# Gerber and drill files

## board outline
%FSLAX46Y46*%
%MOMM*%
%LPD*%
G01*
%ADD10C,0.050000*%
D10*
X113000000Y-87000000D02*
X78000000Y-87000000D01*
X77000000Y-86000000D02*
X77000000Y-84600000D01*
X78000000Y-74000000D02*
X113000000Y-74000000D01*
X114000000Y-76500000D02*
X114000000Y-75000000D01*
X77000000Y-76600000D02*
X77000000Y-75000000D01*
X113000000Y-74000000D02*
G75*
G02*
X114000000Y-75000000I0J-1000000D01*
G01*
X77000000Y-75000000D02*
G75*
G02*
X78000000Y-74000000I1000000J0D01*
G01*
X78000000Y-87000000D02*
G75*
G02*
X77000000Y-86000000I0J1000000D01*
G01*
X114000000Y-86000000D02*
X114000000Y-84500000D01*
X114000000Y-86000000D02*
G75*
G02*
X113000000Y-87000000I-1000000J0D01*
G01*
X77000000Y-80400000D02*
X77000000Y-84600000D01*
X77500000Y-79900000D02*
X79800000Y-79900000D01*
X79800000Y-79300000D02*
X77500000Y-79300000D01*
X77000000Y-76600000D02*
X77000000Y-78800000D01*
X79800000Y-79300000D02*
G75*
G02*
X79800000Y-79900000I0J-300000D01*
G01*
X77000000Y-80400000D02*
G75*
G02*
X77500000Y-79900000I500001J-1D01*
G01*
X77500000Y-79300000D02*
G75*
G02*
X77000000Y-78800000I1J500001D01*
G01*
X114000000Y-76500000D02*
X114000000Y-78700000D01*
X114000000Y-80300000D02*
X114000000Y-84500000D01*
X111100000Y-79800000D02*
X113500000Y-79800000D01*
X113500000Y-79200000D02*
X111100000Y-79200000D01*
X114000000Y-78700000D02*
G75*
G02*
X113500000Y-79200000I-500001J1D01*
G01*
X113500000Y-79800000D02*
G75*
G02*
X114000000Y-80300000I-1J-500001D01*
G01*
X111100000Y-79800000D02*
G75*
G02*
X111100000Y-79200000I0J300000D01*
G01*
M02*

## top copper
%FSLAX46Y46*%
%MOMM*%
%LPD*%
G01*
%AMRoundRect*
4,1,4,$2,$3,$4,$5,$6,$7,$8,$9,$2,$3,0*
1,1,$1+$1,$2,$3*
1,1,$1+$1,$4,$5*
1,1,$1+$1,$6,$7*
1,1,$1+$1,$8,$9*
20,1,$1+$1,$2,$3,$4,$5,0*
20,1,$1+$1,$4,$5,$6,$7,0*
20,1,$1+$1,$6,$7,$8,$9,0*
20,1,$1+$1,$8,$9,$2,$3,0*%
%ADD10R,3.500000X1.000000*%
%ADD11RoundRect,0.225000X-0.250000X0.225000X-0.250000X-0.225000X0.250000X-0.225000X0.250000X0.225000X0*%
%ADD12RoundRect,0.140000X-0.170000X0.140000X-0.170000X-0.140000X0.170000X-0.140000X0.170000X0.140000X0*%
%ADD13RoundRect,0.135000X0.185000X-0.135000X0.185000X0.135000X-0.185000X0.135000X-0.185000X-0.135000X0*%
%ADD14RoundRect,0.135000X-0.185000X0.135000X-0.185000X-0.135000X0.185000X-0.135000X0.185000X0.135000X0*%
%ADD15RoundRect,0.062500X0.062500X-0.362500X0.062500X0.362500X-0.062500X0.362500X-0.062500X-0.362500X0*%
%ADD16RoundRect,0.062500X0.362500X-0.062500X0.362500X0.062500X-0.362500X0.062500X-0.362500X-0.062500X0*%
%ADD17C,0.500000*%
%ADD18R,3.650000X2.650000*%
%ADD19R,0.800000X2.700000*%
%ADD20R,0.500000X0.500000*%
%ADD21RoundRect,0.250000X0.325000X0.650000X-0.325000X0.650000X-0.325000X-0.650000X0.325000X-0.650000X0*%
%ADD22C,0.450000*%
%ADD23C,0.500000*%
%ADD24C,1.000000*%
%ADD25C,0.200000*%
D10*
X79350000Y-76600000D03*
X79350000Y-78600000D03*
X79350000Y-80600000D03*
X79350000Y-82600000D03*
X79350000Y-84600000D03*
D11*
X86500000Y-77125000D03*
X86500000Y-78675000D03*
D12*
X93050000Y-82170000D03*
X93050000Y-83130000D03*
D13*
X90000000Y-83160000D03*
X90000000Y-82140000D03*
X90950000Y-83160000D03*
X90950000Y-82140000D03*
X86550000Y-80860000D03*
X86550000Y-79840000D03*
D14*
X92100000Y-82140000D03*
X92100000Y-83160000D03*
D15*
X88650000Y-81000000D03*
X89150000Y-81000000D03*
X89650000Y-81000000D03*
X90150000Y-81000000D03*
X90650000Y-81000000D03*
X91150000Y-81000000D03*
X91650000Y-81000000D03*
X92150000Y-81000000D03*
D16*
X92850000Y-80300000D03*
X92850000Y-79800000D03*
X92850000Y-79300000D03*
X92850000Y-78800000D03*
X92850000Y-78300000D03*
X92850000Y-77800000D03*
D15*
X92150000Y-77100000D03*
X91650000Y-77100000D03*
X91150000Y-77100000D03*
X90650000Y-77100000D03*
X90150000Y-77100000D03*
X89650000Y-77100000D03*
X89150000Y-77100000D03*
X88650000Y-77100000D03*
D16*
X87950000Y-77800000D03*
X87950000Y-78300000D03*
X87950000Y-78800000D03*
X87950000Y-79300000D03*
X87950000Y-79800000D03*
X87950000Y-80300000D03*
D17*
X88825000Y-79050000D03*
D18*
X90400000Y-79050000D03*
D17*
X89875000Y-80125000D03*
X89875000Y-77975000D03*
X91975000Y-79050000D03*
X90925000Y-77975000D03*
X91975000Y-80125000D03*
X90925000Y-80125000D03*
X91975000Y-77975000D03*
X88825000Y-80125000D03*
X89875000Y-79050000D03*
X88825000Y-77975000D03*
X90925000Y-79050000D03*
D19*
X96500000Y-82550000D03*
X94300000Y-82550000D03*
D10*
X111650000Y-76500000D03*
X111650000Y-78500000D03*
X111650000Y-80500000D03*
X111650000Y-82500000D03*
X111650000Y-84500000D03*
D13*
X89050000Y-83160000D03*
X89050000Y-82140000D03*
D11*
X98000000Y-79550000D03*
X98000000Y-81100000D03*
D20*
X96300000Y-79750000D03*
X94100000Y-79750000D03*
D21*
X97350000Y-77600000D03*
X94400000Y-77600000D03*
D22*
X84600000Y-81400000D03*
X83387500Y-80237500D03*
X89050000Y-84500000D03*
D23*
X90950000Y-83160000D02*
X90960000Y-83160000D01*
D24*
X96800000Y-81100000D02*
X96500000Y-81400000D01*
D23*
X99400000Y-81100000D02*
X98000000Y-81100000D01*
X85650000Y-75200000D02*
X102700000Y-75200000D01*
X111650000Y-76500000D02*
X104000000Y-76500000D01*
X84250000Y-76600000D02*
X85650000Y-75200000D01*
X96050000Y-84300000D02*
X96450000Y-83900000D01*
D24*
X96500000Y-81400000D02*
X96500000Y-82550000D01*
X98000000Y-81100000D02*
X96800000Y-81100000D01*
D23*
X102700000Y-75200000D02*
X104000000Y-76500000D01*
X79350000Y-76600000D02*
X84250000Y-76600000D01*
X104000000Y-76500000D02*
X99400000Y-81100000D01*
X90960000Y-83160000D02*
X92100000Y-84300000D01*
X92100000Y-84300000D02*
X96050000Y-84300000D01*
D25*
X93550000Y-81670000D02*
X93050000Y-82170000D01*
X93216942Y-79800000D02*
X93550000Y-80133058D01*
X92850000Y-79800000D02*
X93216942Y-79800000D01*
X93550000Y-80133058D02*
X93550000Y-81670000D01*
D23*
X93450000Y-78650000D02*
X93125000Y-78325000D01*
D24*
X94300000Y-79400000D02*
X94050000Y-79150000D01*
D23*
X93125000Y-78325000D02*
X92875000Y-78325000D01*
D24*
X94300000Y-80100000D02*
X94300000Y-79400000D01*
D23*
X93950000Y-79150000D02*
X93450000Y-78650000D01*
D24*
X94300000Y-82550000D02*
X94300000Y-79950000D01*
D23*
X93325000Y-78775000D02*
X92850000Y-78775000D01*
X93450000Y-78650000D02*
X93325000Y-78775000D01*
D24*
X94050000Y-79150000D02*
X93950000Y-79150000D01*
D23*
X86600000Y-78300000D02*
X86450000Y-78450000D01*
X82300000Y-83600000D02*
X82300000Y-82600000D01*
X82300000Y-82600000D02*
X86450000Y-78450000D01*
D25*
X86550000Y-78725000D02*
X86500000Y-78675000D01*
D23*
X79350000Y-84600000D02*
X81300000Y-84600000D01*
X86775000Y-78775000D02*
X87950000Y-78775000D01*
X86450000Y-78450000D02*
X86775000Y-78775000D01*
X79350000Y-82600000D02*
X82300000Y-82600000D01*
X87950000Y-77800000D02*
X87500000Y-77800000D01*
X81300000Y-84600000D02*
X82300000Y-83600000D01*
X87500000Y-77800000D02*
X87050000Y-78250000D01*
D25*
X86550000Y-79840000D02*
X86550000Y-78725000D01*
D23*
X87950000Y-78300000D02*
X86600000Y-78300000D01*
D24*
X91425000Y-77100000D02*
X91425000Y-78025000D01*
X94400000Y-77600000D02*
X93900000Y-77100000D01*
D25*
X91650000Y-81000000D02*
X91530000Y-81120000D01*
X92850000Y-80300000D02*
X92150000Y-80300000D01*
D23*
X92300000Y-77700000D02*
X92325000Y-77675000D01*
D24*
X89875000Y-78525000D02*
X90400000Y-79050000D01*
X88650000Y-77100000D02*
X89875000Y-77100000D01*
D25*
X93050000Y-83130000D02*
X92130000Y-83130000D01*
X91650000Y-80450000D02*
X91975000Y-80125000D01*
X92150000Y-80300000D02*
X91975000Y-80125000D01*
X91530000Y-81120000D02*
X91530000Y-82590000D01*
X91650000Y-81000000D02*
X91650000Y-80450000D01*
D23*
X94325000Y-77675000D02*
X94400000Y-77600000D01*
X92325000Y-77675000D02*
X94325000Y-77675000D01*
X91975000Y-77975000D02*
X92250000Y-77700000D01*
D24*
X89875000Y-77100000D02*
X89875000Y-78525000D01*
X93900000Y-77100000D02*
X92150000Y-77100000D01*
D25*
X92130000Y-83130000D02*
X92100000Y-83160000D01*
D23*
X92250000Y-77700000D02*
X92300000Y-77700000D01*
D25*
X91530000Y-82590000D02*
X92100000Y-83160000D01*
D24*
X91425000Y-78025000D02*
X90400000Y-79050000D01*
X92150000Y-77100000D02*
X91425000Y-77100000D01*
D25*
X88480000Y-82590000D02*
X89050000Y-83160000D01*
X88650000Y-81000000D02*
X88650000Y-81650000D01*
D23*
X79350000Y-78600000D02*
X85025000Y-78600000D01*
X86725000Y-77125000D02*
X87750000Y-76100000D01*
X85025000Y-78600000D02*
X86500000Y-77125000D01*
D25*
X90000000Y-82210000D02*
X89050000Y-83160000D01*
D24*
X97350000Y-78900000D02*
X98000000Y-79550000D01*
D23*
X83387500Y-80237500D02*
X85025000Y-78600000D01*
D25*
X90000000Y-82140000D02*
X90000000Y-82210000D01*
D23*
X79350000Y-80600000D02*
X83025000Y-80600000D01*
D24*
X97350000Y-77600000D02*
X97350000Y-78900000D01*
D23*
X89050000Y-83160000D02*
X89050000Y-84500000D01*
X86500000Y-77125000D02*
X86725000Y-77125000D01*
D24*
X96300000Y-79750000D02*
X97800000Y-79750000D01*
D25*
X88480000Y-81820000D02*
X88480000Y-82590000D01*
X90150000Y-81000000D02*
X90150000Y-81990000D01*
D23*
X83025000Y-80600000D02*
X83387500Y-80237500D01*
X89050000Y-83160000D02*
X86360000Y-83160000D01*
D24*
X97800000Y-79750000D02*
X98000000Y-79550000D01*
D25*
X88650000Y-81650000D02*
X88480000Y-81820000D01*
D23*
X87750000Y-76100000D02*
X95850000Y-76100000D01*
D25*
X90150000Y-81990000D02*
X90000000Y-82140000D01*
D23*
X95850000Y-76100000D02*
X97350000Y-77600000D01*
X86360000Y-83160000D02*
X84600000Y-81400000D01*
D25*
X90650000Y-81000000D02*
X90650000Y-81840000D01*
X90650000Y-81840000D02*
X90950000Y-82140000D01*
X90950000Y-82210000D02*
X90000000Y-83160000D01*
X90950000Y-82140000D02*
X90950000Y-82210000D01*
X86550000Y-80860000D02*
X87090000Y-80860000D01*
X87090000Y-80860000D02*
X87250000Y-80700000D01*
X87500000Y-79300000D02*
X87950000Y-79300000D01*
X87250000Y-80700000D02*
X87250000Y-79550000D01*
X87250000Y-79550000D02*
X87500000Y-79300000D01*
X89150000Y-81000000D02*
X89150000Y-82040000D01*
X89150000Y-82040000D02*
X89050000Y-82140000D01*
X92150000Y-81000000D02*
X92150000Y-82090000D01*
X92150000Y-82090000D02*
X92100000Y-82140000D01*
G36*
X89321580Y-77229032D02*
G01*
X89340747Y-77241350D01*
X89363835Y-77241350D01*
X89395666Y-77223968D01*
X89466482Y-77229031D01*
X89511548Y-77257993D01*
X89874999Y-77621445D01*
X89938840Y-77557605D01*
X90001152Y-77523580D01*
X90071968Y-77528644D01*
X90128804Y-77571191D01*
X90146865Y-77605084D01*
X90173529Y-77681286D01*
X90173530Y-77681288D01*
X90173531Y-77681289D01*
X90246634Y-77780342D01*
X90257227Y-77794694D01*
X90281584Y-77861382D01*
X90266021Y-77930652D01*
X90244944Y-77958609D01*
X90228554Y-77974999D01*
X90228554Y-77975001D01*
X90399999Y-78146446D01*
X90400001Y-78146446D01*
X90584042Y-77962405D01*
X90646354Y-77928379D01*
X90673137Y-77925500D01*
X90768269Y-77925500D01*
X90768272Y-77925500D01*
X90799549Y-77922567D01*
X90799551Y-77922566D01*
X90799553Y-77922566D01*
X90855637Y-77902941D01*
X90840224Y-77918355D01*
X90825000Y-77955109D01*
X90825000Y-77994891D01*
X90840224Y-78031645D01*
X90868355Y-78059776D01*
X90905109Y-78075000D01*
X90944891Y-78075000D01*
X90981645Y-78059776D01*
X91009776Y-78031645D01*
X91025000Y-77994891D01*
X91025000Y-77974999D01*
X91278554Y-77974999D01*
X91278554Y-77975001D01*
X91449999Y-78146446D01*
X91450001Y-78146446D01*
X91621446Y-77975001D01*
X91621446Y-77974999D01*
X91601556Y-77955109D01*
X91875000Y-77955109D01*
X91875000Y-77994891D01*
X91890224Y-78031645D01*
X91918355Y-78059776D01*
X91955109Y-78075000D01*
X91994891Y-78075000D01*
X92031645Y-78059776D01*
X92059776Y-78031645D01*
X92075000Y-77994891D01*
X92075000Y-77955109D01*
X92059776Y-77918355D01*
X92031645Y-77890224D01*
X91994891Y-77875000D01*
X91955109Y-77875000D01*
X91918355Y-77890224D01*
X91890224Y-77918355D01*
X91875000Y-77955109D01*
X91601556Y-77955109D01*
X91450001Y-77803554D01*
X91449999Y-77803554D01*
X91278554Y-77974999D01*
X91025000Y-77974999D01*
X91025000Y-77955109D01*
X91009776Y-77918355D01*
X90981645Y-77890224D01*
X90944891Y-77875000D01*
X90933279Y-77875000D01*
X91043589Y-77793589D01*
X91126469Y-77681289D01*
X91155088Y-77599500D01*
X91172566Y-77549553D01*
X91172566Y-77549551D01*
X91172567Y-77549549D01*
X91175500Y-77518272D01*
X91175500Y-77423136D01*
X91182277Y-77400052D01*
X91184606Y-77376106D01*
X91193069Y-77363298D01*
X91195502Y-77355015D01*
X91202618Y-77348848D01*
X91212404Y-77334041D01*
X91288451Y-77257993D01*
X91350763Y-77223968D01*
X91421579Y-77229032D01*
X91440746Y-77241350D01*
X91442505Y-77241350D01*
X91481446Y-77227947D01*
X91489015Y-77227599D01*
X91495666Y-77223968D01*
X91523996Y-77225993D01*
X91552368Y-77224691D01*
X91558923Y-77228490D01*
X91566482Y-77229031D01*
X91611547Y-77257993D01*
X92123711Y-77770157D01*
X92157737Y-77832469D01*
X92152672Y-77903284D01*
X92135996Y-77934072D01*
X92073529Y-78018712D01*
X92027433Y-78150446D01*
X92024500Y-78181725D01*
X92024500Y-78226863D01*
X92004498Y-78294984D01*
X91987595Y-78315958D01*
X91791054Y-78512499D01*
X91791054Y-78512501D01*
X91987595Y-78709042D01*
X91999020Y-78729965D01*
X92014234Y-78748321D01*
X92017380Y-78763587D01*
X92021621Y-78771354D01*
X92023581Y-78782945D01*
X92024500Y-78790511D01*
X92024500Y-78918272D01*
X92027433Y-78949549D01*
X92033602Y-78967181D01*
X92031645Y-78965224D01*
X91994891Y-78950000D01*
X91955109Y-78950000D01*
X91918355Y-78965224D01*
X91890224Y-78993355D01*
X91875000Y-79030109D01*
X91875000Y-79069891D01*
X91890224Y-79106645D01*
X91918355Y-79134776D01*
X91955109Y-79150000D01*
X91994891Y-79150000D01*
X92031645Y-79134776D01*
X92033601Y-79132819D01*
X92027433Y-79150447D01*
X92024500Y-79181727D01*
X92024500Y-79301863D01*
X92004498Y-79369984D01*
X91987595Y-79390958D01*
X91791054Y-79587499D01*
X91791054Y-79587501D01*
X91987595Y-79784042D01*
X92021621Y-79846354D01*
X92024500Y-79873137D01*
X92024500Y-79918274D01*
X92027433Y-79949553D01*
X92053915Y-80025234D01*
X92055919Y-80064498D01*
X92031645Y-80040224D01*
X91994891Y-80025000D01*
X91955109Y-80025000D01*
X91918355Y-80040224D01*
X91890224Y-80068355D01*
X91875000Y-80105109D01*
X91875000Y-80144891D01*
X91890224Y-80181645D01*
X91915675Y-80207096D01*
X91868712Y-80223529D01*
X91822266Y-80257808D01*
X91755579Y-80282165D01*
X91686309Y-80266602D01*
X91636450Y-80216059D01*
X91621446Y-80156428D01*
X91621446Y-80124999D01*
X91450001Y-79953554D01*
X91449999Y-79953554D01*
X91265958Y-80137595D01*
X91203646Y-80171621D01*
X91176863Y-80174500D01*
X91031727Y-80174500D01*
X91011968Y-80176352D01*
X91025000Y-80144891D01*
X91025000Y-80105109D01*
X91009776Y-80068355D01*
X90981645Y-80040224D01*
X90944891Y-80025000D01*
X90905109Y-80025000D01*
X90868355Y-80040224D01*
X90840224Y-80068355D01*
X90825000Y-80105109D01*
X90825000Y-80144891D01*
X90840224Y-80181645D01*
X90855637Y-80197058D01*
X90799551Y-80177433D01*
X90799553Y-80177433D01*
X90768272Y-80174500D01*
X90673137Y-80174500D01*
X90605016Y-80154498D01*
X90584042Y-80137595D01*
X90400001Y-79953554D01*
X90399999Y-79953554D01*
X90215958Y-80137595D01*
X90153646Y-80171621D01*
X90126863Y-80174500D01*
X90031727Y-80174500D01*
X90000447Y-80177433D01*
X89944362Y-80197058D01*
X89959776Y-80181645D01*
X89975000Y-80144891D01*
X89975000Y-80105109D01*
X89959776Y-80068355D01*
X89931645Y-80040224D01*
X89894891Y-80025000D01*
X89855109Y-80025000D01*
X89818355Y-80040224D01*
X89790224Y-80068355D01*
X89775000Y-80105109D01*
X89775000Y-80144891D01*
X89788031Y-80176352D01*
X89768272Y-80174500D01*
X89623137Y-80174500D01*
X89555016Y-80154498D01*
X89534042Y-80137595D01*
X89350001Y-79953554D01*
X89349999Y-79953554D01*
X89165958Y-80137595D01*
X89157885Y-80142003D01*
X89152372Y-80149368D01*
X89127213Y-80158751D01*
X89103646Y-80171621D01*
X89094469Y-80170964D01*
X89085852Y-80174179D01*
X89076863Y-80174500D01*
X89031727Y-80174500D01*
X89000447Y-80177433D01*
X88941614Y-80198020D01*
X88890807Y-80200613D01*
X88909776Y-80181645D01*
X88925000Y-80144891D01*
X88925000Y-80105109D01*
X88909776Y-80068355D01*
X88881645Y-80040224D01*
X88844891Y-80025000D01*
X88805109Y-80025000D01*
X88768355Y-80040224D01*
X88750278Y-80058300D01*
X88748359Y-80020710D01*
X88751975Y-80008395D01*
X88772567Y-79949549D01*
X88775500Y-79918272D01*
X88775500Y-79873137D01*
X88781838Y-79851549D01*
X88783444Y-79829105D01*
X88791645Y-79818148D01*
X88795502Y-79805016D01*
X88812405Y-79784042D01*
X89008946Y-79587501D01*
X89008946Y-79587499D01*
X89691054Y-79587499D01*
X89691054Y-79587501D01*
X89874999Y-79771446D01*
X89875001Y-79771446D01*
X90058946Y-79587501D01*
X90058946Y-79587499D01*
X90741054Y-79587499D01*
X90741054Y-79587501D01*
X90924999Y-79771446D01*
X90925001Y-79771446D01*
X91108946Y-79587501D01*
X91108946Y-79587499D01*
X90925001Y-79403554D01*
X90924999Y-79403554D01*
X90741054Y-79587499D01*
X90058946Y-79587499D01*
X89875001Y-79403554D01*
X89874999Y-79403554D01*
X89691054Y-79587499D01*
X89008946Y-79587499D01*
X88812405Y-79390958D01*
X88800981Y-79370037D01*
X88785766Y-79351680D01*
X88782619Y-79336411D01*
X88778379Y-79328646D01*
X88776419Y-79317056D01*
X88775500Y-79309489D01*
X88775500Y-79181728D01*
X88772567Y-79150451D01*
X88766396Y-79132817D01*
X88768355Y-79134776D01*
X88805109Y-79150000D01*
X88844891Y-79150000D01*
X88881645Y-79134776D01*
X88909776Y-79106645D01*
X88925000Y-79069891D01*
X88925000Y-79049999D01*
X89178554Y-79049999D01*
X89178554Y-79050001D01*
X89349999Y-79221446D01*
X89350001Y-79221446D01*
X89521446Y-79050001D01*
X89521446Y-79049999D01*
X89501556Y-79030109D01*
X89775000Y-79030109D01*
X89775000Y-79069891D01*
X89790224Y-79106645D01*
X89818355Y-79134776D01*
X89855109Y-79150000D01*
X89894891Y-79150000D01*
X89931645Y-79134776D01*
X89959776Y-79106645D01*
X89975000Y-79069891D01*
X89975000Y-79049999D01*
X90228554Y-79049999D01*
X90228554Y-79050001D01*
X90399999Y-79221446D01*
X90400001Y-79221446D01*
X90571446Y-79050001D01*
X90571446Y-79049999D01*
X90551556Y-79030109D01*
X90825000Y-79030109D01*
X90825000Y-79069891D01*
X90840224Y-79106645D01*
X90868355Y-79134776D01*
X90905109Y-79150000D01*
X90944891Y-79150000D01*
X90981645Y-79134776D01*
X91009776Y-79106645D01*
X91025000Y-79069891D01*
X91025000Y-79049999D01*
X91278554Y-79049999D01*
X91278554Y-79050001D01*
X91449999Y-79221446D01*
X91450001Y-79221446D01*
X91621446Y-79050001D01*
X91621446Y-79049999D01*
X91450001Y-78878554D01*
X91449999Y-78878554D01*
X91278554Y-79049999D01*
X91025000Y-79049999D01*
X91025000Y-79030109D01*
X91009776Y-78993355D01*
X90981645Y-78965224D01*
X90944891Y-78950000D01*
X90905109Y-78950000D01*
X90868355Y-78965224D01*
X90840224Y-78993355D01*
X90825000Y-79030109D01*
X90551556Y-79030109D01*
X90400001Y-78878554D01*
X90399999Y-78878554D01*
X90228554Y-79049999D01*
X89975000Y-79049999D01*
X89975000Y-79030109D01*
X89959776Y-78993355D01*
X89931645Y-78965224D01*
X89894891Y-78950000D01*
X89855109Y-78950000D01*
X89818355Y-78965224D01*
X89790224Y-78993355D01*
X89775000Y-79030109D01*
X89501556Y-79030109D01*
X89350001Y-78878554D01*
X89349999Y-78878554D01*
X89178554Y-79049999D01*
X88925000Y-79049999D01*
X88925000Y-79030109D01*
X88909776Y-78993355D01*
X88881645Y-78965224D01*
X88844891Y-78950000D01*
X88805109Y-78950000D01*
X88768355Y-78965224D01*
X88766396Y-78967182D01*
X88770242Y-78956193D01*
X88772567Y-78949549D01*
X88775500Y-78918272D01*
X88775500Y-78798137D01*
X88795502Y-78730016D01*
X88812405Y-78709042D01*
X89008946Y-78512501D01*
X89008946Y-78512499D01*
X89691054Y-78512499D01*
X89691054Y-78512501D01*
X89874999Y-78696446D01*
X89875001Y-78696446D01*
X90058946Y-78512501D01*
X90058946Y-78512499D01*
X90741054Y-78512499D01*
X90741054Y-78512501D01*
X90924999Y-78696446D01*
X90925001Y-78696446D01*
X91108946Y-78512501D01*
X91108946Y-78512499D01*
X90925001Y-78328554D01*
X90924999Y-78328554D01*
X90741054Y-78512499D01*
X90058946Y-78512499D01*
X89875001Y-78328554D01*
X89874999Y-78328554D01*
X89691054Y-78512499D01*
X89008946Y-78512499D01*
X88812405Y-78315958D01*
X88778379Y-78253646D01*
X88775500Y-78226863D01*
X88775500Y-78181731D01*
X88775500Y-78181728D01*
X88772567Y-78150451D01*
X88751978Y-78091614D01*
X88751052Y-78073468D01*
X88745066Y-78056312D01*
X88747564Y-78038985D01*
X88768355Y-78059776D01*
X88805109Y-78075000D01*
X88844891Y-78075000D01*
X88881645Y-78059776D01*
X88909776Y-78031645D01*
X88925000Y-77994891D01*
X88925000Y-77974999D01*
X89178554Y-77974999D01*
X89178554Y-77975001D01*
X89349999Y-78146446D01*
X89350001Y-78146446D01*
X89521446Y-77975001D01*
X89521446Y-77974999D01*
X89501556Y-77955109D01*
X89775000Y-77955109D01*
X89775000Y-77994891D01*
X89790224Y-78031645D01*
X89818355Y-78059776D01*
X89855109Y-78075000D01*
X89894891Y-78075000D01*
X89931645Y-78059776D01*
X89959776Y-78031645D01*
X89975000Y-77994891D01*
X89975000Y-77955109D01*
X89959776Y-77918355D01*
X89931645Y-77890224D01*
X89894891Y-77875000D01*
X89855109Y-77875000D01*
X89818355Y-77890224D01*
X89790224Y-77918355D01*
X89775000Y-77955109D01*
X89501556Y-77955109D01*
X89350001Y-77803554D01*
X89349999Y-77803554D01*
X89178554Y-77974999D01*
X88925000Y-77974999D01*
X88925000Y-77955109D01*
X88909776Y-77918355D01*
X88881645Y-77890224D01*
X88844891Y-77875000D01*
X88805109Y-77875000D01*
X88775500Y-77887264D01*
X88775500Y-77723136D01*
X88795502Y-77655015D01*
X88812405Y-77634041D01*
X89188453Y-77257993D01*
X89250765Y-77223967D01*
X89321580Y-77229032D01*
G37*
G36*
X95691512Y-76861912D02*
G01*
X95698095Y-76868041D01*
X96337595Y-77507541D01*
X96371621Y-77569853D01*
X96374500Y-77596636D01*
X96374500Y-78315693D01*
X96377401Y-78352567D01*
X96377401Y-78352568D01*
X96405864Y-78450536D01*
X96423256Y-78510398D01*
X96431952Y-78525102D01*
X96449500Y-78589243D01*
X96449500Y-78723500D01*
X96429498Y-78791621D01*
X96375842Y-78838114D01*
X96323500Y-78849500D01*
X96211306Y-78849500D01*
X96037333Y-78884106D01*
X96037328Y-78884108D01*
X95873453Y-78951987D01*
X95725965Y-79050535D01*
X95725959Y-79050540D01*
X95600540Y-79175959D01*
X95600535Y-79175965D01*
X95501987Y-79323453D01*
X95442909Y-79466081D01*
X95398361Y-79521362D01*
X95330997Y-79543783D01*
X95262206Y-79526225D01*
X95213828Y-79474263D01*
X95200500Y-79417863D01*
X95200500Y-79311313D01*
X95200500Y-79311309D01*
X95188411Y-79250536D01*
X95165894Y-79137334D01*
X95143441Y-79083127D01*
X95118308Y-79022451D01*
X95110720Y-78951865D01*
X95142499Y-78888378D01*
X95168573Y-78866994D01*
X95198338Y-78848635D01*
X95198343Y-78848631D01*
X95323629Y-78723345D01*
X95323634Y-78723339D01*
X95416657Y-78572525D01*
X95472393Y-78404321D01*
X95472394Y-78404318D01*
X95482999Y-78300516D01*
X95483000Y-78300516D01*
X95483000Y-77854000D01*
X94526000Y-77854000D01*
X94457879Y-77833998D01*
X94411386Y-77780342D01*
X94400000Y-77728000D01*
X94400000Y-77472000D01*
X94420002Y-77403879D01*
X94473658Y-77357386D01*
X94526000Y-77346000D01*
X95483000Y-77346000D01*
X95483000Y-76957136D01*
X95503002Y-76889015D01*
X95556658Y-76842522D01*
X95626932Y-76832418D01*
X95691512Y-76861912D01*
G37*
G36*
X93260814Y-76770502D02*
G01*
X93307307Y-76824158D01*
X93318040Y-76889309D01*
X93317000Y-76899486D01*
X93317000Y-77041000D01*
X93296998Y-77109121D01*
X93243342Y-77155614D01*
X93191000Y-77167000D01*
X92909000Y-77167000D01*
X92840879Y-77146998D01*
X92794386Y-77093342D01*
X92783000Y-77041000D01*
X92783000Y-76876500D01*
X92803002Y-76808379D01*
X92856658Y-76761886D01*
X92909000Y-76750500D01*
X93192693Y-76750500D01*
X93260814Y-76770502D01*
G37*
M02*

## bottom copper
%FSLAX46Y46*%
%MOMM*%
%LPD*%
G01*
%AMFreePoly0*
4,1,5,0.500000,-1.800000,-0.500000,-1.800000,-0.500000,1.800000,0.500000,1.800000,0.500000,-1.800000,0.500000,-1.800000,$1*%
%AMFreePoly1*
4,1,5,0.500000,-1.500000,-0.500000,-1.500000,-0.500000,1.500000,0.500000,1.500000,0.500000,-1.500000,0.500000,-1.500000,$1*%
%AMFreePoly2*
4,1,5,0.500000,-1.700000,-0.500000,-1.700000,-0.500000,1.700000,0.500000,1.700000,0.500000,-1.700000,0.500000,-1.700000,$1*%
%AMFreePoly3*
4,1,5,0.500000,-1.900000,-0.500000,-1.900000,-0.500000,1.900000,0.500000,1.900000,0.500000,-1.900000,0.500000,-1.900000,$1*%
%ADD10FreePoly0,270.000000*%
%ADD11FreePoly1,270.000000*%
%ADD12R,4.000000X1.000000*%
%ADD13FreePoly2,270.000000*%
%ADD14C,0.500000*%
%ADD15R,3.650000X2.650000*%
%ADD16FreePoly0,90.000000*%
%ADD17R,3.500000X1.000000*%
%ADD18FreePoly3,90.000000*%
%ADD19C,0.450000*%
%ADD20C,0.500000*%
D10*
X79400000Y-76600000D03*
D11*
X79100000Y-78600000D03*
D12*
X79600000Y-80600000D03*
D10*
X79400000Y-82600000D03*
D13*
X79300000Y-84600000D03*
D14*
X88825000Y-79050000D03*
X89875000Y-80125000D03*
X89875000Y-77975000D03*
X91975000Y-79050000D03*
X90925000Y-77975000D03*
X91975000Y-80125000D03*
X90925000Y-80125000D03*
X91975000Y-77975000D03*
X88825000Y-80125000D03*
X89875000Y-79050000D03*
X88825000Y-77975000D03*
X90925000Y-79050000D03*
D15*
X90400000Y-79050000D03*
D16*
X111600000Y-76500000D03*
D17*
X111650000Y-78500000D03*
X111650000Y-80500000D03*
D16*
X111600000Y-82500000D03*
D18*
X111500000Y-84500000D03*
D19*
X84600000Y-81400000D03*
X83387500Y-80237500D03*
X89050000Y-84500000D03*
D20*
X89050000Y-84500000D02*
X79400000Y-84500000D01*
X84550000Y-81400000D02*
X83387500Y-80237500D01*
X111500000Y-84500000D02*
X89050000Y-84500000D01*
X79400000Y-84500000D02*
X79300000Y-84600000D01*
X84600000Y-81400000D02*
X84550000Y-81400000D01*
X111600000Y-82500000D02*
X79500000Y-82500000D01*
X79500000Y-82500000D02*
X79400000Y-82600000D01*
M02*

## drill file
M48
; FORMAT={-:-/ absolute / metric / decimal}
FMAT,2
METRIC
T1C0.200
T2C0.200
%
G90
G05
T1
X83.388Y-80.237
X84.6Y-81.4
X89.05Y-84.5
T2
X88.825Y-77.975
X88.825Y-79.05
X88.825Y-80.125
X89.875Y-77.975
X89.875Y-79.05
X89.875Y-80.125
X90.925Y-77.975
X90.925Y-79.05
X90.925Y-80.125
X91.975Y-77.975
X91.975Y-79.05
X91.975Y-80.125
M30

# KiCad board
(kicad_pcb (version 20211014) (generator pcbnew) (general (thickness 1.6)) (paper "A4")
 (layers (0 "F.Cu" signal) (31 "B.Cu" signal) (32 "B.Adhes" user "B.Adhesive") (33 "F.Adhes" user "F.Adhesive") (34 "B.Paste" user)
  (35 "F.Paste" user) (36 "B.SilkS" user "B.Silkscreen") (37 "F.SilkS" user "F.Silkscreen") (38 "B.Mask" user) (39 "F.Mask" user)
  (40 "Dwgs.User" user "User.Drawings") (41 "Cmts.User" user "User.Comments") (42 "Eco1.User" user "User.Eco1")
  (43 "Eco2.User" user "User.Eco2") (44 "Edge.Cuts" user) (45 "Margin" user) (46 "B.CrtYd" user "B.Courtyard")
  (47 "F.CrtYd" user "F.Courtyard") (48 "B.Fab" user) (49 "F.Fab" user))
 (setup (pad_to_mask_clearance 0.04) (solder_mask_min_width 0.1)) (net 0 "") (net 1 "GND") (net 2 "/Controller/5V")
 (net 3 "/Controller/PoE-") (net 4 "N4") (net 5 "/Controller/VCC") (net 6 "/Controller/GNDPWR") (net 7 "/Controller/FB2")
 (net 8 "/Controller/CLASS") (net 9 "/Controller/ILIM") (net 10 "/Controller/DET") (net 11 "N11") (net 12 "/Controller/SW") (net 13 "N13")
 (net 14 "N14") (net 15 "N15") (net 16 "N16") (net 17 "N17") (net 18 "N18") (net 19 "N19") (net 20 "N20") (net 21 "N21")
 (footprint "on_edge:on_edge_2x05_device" (layer "F.Cu") (at 77 80.6 -90)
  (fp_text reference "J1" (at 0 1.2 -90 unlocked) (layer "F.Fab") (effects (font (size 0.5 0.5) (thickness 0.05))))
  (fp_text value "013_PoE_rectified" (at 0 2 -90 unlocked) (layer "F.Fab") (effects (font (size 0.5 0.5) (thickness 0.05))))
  (fp_line (start -0.2 0) (end 4 0) (layer "Edge.Cuts") (width 0.05))
  (fp_line (start -0.7 -0.5) (end -0.7 -2.8) (layer "Edge.Cuts") (width 0.05))
  (fp_line (start -1.3 -2.8) (end -1.3 -0.5) (layer "Edge.Cuts") (width 0.05))
  (fp_line (start -4 0) (end -1.8 0) (layer "Edge.Cuts") (width 0.05))
  (fp_arc (start -1.3 -2.8) (mid -1 -3.1) (end -0.7 -2.8) (layer "Edge.Cuts") (width 0.05))
  (fp_arc (start -0.2 0) (mid -0.553553 -0.146447) (end -0.7 -0.5) (layer "Edge.Cuts") (width 0.05))
  (fp_arc (start -1.3 -0.5) (mid -1.446447 -0.146447) (end -1.8 0) (layer "Edge.Cuts") (width 0.05))
  (pad "1" smd rect (at -4 -2.35 90) (size 1 3.5) (layers "F.Cu" "F.Mask") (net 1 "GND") (zone_connect 0))
  (pad "2" smd rect (at -2 -2.35 270) (size 1 3.5) (layers "F.Cu" "F.Mask") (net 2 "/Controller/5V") (zone_connect 0))
  (pad "3" smd rect (at 0 -2.35 270) (size 1 3.5) (layers "F.Cu" "F.Mask") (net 2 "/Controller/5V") (zone_connect 0))
  (pad "4" smd rect (at 2 -2.35 90) (size 1 3.5) (layers "F.Cu" "F.Mask") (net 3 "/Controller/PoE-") (zone_connect 0))
  (pad "5" smd rect (at 4 -2.35 90) (size 1 3.5) (layers "F.Cu" "F.Mask") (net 3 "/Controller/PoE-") (zone_connect 0))
  (pad "6" smd custom (at -4 -2.4 270) (size 1 3.6) (layers "B.Cu" "B.Mask") (zone_connect 0) (options (clearance outline) (anchor rect))
   (primitives))
  (pad "7" smd custom (at -2 -2.1 270) (size 1 3) (layers "B.Cu" "B.Mask") (zone_connect 0) (options (clearance outline) (anchor rect))
   (primitives))
  (pad "8" smd rect (at 0 -2.6 270) (size 1 4) (layers "B.Cu" "B.Mask") (zone_connect 0))
  (pad "9" smd custom (at 2 -2.4 270) (size 1 3.6) (layers "B.Cu" "B.Mask") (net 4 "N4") (zone_connect 0)
   (options (clearance outline) (anchor rect)) (primitives))
  (pad "10" smd custom (at 4 -2.3 270) (size 1 3.4) (layers "B.Cu" "B.Mask") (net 2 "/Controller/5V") (zone_connect 0)
   (options (clearance outline) (anchor rect)) (primitives))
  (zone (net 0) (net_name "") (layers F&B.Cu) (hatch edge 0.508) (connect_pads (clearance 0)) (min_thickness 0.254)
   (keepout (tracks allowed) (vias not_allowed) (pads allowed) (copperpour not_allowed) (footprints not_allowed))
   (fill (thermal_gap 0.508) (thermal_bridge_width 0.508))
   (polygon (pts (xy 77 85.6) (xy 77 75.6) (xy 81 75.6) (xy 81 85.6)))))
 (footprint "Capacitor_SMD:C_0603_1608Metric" (layer "F.Cu") (at 86.5 77.9 -90)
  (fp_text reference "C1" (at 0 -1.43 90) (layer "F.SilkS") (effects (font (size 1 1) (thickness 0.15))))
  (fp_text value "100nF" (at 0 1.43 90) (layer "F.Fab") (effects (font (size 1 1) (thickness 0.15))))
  (pad "1" smd roundrect (at -0.775 0 270) (size 0.9 0.95) (layers "F.Cu" "F.Paste" "F.Mask") (roundrect_rratio 0.25)
   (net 2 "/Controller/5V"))
  (pad "2" smd roundrect (at 0.775 0 270) (size 0.9 0.95) (layers "F.Cu" "F.Paste" "F.Mask") (roundrect_rratio 0.25)
   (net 3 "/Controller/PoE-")))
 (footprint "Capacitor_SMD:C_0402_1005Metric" (layer "F.Cu") (at 93.05 82.65 -90)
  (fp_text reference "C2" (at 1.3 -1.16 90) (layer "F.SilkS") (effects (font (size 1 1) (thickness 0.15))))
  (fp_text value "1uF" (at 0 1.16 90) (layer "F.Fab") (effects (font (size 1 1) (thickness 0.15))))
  (pad "1" smd roundrect (at -0.48 0 270) (size 0.56 0.62) (layers "F.Cu" "F.Paste" "F.Mask") (roundrect_rratio 0.25)
   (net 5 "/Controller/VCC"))
  (pad "2" smd roundrect (at 0.48 0 270) (size 0.56 0.62) (layers "F.Cu" "F.Paste" "F.Mask") (roundrect_rratio 0.25)
   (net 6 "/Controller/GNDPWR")))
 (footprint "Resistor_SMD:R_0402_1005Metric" (layer "F.Cu") (at 90 82.65 90)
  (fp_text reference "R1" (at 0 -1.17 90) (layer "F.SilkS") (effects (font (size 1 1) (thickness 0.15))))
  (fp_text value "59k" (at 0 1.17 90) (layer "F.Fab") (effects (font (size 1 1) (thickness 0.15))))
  (pad "1" smd roundrect (at -0.51 0 90) (size 0.54 0.64) (layers "F.Cu" "F.Paste" "F.Mask") (roundrect_rratio 0.25)
   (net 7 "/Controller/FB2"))
  (pad "2" smd roundrect (at 0.51 0 90) (size 0.54 0.64) (layers "F.Cu" "F.Paste" "F.Mask") (roundrect_rratio 0.25) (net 2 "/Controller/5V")))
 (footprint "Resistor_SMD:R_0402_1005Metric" (layer "F.Cu") (at 90.95 82.65 90)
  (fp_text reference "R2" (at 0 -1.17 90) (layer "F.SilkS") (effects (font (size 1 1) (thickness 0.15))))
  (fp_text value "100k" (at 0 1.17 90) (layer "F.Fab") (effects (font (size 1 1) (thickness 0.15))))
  (pad "1" smd roundrect (at -0.51 0 90) (size 0.54 0.64) (layers "F.Cu" "F.Paste" "F.Mask") (roundrect_rratio 0.25) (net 1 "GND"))
  (pad "2" smd roundrect (at 0.51 0 90) (size 0.54 0.64) (layers "F.Cu" "F.Paste" "F.Mask") (roundrect_rratio 0.25)
   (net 7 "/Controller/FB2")))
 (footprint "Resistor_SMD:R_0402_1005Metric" (layer "F.Cu") (at 86.55 80.35 90)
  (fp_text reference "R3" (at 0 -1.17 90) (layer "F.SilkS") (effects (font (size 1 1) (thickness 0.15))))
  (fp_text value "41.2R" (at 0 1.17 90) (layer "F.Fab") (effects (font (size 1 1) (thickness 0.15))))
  (pad "1" smd roundrect (at -0.51 0 90) (size 0.54 0.64) (layers "F.Cu" "F.Paste" "F.Mask") (roundrect_rratio 0.25)
   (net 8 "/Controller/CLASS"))
  (pad "2" smd roundrect (at 0.51 0 90) (size 0.54 0.64) (layers "F.Cu" "F.Paste" "F.Mask") (roundrect_rratio 0.25)
   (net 3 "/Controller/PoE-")))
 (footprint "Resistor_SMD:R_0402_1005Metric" (layer "F.Cu") (at 92.1 82.65 -90)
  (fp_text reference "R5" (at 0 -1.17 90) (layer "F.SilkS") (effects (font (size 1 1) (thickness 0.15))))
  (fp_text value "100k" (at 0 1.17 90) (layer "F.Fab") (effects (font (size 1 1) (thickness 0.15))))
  (pad "1" smd roundrect (at -0.51 0 270) (size 0.54 0.64) (layers "F.Cu" "F.Paste" "F.Mask") (roundrect_rratio 0.25)
   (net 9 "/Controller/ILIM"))
  (pad "2" smd roundrect (at 0.51 0 270) (size 0.54 0.64) (layers "F.Cu" "F.Paste" "F.Mask") (roundrect_rratio 0.25)
   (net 6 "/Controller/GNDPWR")))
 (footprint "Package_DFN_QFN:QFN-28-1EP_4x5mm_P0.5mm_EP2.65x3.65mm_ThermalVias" (layer "F.Cu") (at 90.4 79.05 90)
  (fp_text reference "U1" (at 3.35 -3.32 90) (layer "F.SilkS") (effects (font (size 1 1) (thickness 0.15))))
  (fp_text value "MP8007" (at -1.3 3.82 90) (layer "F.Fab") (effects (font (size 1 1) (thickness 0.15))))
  (pad "" smd roundrect (at 0.66 0 90) (size 1.07 0.98) (layers "F.Paste") (roundrect_rratio 0.25))
  (pad "" smd roundrect (at -0.66 -1.22 90) (size 1.07 0.98) (layers "F.Paste") (roundrect_rratio 0.25))
  (pad "" smd roundrect (at -0.66 1.22 90) (size 1.07 0.98) (layers "F.Paste") (roundrect_rratio 0.25))
  (pad "" smd roundrect (at 0.66 1.22 90) (size 1.07 0.98) (layers "F.Paste") (roundrect_rratio 0.25))
  (pad "" smd roundrect (at -0.66 0 90) (size 1.07 0.98) (layers "F.Paste") (roundrect_rratio 0.25))
  (pad "" smd roundrect (at 0.66 -1.22 90) (size 1.07 0.98) (layers "F.Paste") (roundrect_rratio 0.25))
  (pad "1" smd roundrect (at -1.95 -1.75 90) (size 0.85 0.25) (layers "F.Cu" "F.Paste" "F.Mask") (roundrect_rratio 0.25)
   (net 2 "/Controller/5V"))
  (pad "2" smd roundrect (at -1.95 -1.25 90) (size 0.85 0.25) (layers "F.Cu" "F.Paste" "F.Mask") (roundrect_rratio 0.25)
   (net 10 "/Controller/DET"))
  (pad "3" smd roundrect (at -1.95 -0.75 90) (size 0.85 0.25) (layers "F.Cu" "F.Paste" "F.Mask") (roundrect_rratio 0.25))
  (pad "4" smd roundrect (at -1.95 -0.25 90) (size 0.85 0.25) (layers "F.Cu" "F.Paste" "F.Mask") (roundrect_rratio 0.25)
   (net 2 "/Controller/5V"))
  (pad "5" smd roundrect (at -1.95 0.25 90) (size 0.85 0.25) (layers "F.Cu" "F.Paste" "F.Mask") (roundrect_rratio 0.25)
   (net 7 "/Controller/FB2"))
  (pad "6" smd roundrect (at -1.95 0.75 90) (size 0.85 0.25) (layers "F.Cu" "F.Paste" "F.Mask") (roundrect_rratio 0.25) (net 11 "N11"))
  (pad "7" smd roundrect (at -1.95 1.25 90) (size 0.85 0.25) (layers "F.Cu" "F.Paste" "F.Mask") (roundrect_rratio 0.25)
   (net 6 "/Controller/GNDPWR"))
  (pad "8" smd roundrect (at -1.95 1.75 90) (size 0.85 0.25) (layers "F.Cu" "F.Paste" "F.Mask") (roundrect_rratio 0.25)
   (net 9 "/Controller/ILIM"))
  (pad "9" smd roundrect (at -1.25 2.45 90) (size 0.25 0.85) (layers "F.Cu" "F.Paste" "F.Mask") (roundrect_rratio 0.25)
   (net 6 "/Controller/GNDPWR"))
  (pad "10" smd roundrect (at -0.75 2.45 90) (size 0.25 0.85) (layers "F.Cu" "F.Paste" "F.Mask") (roundrect_rratio 0.25)
   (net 5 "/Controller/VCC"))
  (pad "11" smd roundrect (at -0.25 2.45 90) (size 0.25 0.85) (layers "F.Cu" "F.Paste" "F.Mask") (roundrect_rratio 0.25))
  (pad "12" smd roundrect (at 0.25 2.45 90) (size 0.25 0.85) (layers "F.Cu" "F.Paste" "F.Mask") (roundrect_rratio 0.25)
   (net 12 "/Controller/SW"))
  (pad "13" smd roundrect (at 0.75 2.45 90) (size 0.25 0.85) (layers "F.Cu" "F.Paste" "F.Mask") (roundrect_rratio 0.25)
   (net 12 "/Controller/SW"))
  (pad "14" smd roundrect (at 1.25 2.45 90) (size 0.25 0.85) (layers "F.Cu" "F.Paste" "F.Mask") (roundrect_rratio 0.25)
   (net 6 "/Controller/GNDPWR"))
  (pad "15" smd roundrect (at 1.95 1.75 90) (size 0.85 0.25) (layers "F.Cu" "F.Paste" "F.Mask") (roundrect_rratio 0.25)
   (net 6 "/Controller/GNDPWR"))
  (pad "16" smd roundrect (at 1.95 1.25 90) (size 0.85 0.25) (layers "F.Cu" "F.Paste" "F.Mask") (roundrect_rratio 0.25)
   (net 6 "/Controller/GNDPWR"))
  (pad "17" smd roundrect (at 1.95 0.75 90) (size 0.85 0.25) (layers "F.Cu" "F.Paste" "F.Mask") (roundrect_rratio 0.25)
   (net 6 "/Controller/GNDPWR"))
  (pad "18" smd roundrect (at 1.95 0.25 90) (size 0.85 0.25) (layers "F.Cu" "F.Paste" "F.Mask") (roundrect_rratio 0.25) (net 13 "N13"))
  (pad "19" smd roundrect (at 1.95 -0.25 90) (size 0.85 0.25) (layers "F.Cu" "F.Paste" "F.Mask") (roundrect_rratio 0.25)
   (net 6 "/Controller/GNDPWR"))
  (pad "20" smd roundrect (at 1.95 -0.75 90) (size 0.85 0.25) (layers "F.Cu" "F.Paste" "F.Mask") (roundrect_rratio 0.25)
   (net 6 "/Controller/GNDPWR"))
  (pad "21" smd roundrect (at 1.95 -1.25 90) (size 0.85 0.25) (layers "F.Cu" "F.Paste" "F.Mask") (roundrect_rratio 0.25)
   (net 6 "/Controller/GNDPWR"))
  (pad "22" smd roundrect (at 1.95 -1.75 90) (size 0.85 0.25) (layers "F.Cu" "F.Paste" "F.Mask") (roundrect_rratio 0.25)
   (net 6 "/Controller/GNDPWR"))
  (pad "23" smd roundrect (at 1.25 -2.45 90) (size 0.25 0.85) (layers "F.Cu" "F.Paste" "F.Mask") (roundrect_rratio 0.25)
   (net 3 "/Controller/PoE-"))
  (pad "24" smd roundrect (at 0.75 -2.45 90) (size 0.25 0.85) (layers "F.Cu" "F.Paste" "F.Mask") (roundrect_rratio 0.25)
   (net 3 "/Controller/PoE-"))
  (pad "25" smd roundrect (at 0.25 -2.45 90) (size 0.25 0.85) (layers "F.Cu" "F.Paste" "F.Mask") (roundrect_rratio 0.25)
   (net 3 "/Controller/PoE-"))
  (pad "26" smd roundrect (at -0.25 -2.45 90) (size 0.25 0.85) (layers "F.Cu" "F.Paste" "F.Mask") (roundrect_rratio 0.25)
   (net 8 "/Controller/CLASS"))
  (pad "27" smd roundrect (at -0.75 -2.45 90) (size 0.25 0.85) (layers "F.Cu" "F.Paste" "F.Mask") (roundrect_rratio 0.25) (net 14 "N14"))
  (pad "28" smd roundrect (at -1.25 -2.45 90) (size 0.25 0.85) (layers "F.Cu" "F.Paste" "F.Mask") (roundrect_rratio 0.25))
  (pad "29" thru_hole circle (at 0 -1.575 90) (size 0.5 0.5) (drill 0.2) (layers *.Cu) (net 6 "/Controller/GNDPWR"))
  (pad "29" smd rect (at 0 0 90) (size 2.65 3.65) (layers "F.Cu" "F.Mask") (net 6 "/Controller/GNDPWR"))
  (pad "29" thru_hole circle (at -1.075 -0.525 90) (size 0.5 0.5) (drill 0.2) (layers *.Cu) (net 6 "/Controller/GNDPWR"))
  (pad "29" thru_hole circle (at 1.075 -0.525 90) (size 0.5 0.5) (drill 0.2) (layers *.Cu) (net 6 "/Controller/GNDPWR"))
  (pad "29" thru_hole circle (at 0 1.575 90) (size 0.5 0.5) (drill 0.2) (layers *.Cu) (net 6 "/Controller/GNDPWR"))
  (pad "29" thru_hole circle (at 1.075 0.525 90) (size 0.5 0.5) (drill 0.2) (layers *.Cu) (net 6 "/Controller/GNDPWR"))
  (pad "29" thru_hole circle (at -1.075 1.575 90) (size 0.5 0.5) (drill 0.2) (layers *.Cu) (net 6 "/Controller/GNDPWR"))
  (pad "29" thru_hole circle (at -1.075 0.525 90) (size 0.5 0.5) (drill 0.2) (layers *.Cu) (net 6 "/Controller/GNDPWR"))
  (pad "29" thru_hole circle (at 1.075 1.575 90) (size 0.5 0.5) (drill 0.2) (layers *.Cu) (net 6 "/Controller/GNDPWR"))
  (pad "29" thru_hole circle (at -1.075 -1.575 90) (size 0.5 0.5) (drill 0.2) (layers *.Cu) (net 6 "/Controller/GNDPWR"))
  (pad "29" thru_hole circle (at 0 -0.525 90) (size 0.5 0.5) (drill 0.2) (layers *.Cu) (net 6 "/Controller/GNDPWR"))
  (pad "29" thru_hole circle (at 1.075 -1.575 90) (size 0.5 0.5) (drill 0.2) (layers *.Cu) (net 6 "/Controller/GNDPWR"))
  (pad "29" thru_hole circle (at 0 0.525 90) (size 0.5 0.5) (drill 0.2) (layers *.Cu) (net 6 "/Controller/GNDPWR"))
  (pad "29" smd rect (at 0 0 90) (size 2.65 3.65) (layers "B.Cu") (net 6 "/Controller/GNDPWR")))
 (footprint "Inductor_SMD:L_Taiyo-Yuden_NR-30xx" (layer "F.Cu") (at 95.4 82.55 180)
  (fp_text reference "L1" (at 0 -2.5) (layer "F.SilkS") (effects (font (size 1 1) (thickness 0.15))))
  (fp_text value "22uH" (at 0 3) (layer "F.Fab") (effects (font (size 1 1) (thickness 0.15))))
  (pad "1" smd rect (at -1.1 0 180) (size 0.8 2.7) (layers "F.Cu" "F.Paste" "F.Mask") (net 1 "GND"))
  (pad "2" smd rect (at 1.1 0 180) (size 0.8 2.7) (layers "F.Cu" "F.Paste" "F.Mask") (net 12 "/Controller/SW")))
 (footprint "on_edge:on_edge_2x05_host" (layer "F.Cu") (at 114 80.5 -90)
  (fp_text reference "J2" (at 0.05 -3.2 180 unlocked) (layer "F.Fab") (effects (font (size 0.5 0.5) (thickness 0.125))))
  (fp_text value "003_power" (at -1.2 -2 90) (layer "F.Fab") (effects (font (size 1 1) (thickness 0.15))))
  (fp_line (start -4 0) (end -1.8 0) (layer "Edge.Cuts") (width 0.05))
  (fp_line (start -0.2 0) (end 4 0) (layer "Edge.Cuts") (width 0.05))
  (fp_line (start -0.7 2.9) (end -0.7 0.5) (layer "Edge.Cuts") (width 0.05))
  (fp_line (start -1.3 0.5) (end -1.3 2.9) (layer "Edge.Cuts") (width 0.05))
  (fp_arc (start -1.8 0) (mid -1.446447 0.146447) (end -1.3 0.5) (layer "Edge.Cuts") (width 0.05))
  (fp_arc (start -0.7 0.5) (mid -0.553553 0.146447) (end -0.2 0) (layer "Edge.Cuts") (width 0.05))
  (fp_arc (start -0.7 2.9) (mid -1 3.2) (end -1.3 2.9) (layer "Edge.Cuts") (width 0.05))
  (pad "1" smd rect (at -4 2.35 270) (size 1 3.5) (layers "F.Cu" "F.Mask") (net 1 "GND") (zone_connect 0))
  (pad "2" smd rect (at -2 2.35 270) (size 1 3.5) (layers "F.Cu" "F.Mask") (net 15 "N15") (zone_connect 0))
  (pad "3" smd rect (at 0 2.35 270) (size 1 3.5) (layers "F.Cu" "F.Mask") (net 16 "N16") (zone_connect 0))
  (pad "4" smd rect (at 2 2.35 270) (size 1 3.5) (layers "F.Cu" "F.Mask") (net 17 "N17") (zone_connect 0))
  (pad "5" smd rect (at 4 2.35 270) (size 1 3.5) (layers "F.Cu" "F.Mask") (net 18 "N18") (zone_connect 0))
  (pad "6" smd custom (at -4 2.4 90) (size 1 3.6) (layers "B.Cu" "B.Mask") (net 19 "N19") (zone_connect 0)
   (options (clearance outline) (anchor rect)) (primitives))
  (pad "7" smd rect (at -2 2.35 90) (size 1 3.5) (layers "B.Cu" "B.Mask") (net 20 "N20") (zone_connect 0))
  (pad "8" smd rect (at 0 2.35 90) (size 1 3.5) (layers "B.Cu" "B.Mask") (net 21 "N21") (zone_connect 0))
  (pad "9" smd custom (at 2 2.4 90) (size 1 3.6) (layers "B.Cu" "B.Mask") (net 4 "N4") (zone_connect 0)
   (options (clearance outline) (anchor rect)) (primitives))
  (pad "10" smd custom (at 4 2.5 90) (size 1 3.8) (layers "B.Cu" "B.Mask") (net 2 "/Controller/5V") (zone_connect 0)
   (options (clearance outline) (anchor rect)) (primitives))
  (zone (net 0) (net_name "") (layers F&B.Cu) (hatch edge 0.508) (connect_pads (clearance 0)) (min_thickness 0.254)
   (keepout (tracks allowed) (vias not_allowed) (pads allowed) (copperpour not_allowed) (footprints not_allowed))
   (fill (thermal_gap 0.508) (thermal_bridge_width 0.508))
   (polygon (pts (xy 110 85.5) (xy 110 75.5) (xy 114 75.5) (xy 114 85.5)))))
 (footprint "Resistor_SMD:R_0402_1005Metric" (layer "F.Cu") (at 89.05 82.65 90)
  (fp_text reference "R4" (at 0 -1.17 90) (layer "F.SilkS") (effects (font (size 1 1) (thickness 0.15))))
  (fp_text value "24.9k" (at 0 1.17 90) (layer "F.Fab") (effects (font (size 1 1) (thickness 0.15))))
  (pad "1" smd roundrect (at -0.51 0 90) (size 0.54 0.64) (layers "F.Cu" "F.Paste" "F.Mask") (roundrect_rratio 0.25)
   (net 2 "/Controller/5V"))
  (pad "2" smd roundrect (at 0.51 0 90) (size 0.54 0.64) (layers "F.Cu" "F.Paste" "F.Mask") (roundrect_rratio 0.25)
   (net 10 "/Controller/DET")))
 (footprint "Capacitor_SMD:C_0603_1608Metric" (layer "F.Cu") (at 98 80.325 -90)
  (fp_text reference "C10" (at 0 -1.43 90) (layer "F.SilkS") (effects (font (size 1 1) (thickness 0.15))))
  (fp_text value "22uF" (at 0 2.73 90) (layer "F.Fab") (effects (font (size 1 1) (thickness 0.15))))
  (pad "1" smd roundrect (at -0.775 0 270) (size 0.9 0.95) (layers "F.Cu" "F.Paste" "F.Mask") (roundrect_rratio 0.25)
   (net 2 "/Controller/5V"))
  (pad "2" smd roundrect (at 0.775 0 270) (size 0.9 0.95) (layers "F.Cu" "F.Paste" "F.Mask") (roundrect_rratio 0.25) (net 1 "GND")))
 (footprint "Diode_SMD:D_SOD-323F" (layer "F.Cu") (at 95.2 79.75 180)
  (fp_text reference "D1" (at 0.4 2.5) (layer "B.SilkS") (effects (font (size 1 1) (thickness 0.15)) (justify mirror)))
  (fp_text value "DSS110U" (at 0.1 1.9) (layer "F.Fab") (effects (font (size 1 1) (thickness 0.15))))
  (pad "1" smd rect (at -1.1 0 180) (size 0.5 0.5) (layers "F.Cu" "F.Paste" "F.Mask") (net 2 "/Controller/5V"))
  (pad "2" smd rect (at 1.1 0 180) (size 0.5 0.5) (layers "F.Cu" "F.Paste" "F.Mask") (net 12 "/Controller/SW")))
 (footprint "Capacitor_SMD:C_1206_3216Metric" (layer "F.Cu") (at 95.875 77.6 180)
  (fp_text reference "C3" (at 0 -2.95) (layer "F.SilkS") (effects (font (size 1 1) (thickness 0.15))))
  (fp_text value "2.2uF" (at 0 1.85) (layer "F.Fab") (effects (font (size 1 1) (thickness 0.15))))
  (pad "1" smd roundrect (at -1.475 0 180) (size 1.15 1.8) (layers "F.Cu" "F.Paste" "F.Mask") (roundrect_rratio 0.217391)
   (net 2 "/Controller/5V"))
  (pad "2" smd roundrect (at 1.475 0 180) (size 1.15 1.8) (layers "F.Cu" "F.Paste" "F.Mask") (roundrect_rratio 0.217391)
   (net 6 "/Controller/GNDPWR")))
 (gr_line (start 113 87) (end 78 87) (layer "Edge.Cuts") (width 0.05))
 (gr_line (start 77 86) (end 77 84.6) (layer "Edge.Cuts") (width 0.05))
 (gr_line (start 78 74) (end 113 74) (layer "Edge.Cuts") (width 0.05))
 (gr_line (start 114 76.5) (end 114 75) (layer "Edge.Cuts") (width 0.05))
 (gr_line (start 77 76.6) (end 77 75) (layer "Edge.Cuts") (width 0.05))
 (gr_arc (start 113 74) (mid 113.707107 74.292893) (end 114 75) (layer "Edge.Cuts") (width 0.05))
 (gr_arc (start 77 75) (mid 77.292893 74.292893) (end 78 74) (layer "Edge.Cuts") (width 0.05))
 (gr_arc (start 78 87) (mid 77.292893 86.707107) (end 77 86) (layer "Edge.Cuts") (width 0.05))
 (gr_line (start 114 86) (end 114 84.5) (layer "Edge.Cuts") (width 0.05))
 (gr_arc (start 114 86) (mid 113.707107 86.707107) (end 113 87) (layer "Edge.Cuts") (width 0.05))
 (segment (start 90.95 83.16) (end 90.96 83.16) (width 0.5) (layer "F.Cu") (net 1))
 (segment (start 96.8 81.1) (end 96.5 81.4) (width 1) (layer "F.Cu") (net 1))
 (segment (start 99.4 81.1) (end 98 81.1) (width 0.5) (layer "F.Cu") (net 1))
 (segment (start 85.65 75.2) (end 102.7 75.2) (width 0.5) (layer "F.Cu") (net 1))
 (segment (start 111.65 76.5) (end 104 76.5) (width 0.5) (layer "F.Cu") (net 1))
 (segment (start 84.25 76.6) (end 85.65 75.2) (width 0.5) (layer "F.Cu") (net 1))
 (segment (start 96.05 84.3) (end 96.45 83.9) (width 0.5) (layer "F.Cu") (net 1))
 (segment (start 96.5 81.4) (end 96.5 82.55) (width 1) (layer "F.Cu") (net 1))
 (segment (start 98 81.1) (end 96.8 81.1) (width 1) (layer "F.Cu") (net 1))
 (segment (start 102.7 75.2) (end 104 76.5) (width 0.5) (layer "F.Cu") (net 1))
 (segment (start 79.35 76.6) (end 84.25 76.6) (width 0.5) (layer "F.Cu") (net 1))
 (segment (start 104 76.5) (end 99.4 81.1) (width 0.5) (layer "F.Cu") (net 1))
 (segment (start 90.96 83.16) (end 92.1 84.3) (width 0.5) (layer "F.Cu") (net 1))
 (segment (start 92.1 84.3) (end 96.05 84.3) (width 0.5) (layer "F.Cu") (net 1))
 (segment (start 93.55 81.67) (end 93.05 82.17) (width 0.2) (layer "F.Cu") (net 5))
 (segment (start 93.216942 79.8) (end 93.55 80.133058) (width 0.2) (layer "F.Cu") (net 5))
 (segment (start 92.85 79.8) (end 93.216942 79.8) (width 0.2) (layer "F.Cu") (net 5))
 (segment (start 93.55 80.133058) (end 93.55 81.67) (width 0.2) (layer "F.Cu") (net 5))
 (segment (start 93.45 78.65) (end 93.125 78.325) (width 0.5) (layer "F.Cu") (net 12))
 (segment (start 94.3 79.4) (end 94.05 79.15) (width 1) (layer "F.Cu") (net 12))
 (segment (start 93.125 78.325) (end 92.875 78.325) (width 0.5) (layer "F.Cu") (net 12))
 (segment (start 94.3 80.1) (end 94.3 79.4) (width 1) (layer "F.Cu") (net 12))
 (segment (start 93.95 79.15) (end 93.45 78.65) (width 0.5) (layer "F.Cu") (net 12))
 (segment (start 94.3 82.55) (end 94.3 79.95) (width 1) (layer "F.Cu") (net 12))
 (segment (start 93.325 78.775) (end 92.85 78.775) (width 0.5) (layer "F.Cu") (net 12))
 (segment (start 93.45 78.65) (end 93.325 78.775) (width 0.5) (layer "F.Cu") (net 12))
 (segment (start 94.05 79.15) (end 93.95 79.15) (width 1) (layer "F.Cu") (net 12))
 (segment (start 86.6 78.3) (end 86.45 78.45) (width 0.5) (layer "F.Cu") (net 3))
 (segment (start 82.3 83.6) (end 82.3 82.6) (width 0.5) (layer "F.Cu") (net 3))
 (segment (start 82.3 82.6) (end 86.45 78.45) (width 0.5) (layer "F.Cu") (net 3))
 (segment (start 86.55 78.725) (end 86.5 78.675) (width 0.2) (layer "F.Cu") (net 3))
 (segment (start 79.35 84.6) (end 81.3 84.6) (width 0.5) (layer "F.Cu") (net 3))
 (segment (start 86.775 78.775) (end 87.95 78.775) (width 0.5) (layer "F.Cu") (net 3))
 (segment (start 86.45 78.45) (end 86.775 78.775) (width 0.5) (layer "F.Cu") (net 3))
 (segment (start 79.35 82.6) (end 82.3 82.6) (width 0.5) (layer "F.Cu") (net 3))
 (segment (start 87.95 77.8) (end 87.5 77.8) (width 0.5) (layer "F.Cu") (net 3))
 (segment (start 81.3 84.6) (end 82.3 83.6) (width 0.5) (layer "F.Cu") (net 3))
 (segment (start 87.5 77.8) (end 87.05 78.25) (width 0.5) (layer "F.Cu") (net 3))
 (segment (start 86.55 79.84) (end 86.55 78.725) (width 0.2) (layer "F.Cu") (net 3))
 (segment (start 87.95 78.3) (end 86.6 78.3) (width 0.5) (layer "F.Cu") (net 3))
 (segment (start 91.425 77.1) (end 91.425 78.025) (width 1) (layer "F.Cu") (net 6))
 (segment (start 94.4 77.6) (end 93.9 77.1) (width 1) (layer "F.Cu") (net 6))
 (segment (start 91.65 81) (end 91.53 81.12) (width 0.2) (layer "F.Cu") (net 6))
 (segment (start 92.85 80.3) (end 92.15 80.3) (width 0.2) (layer "F.Cu") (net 6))
 (segment (start 92.3 77.7) (end 92.325 77.675) (width 0.5) (layer "F.Cu") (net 6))
 (segment (start 89.875 78.525) (end 90.4 79.05) (width 1) (layer "F.Cu") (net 6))
 (segment (start 88.65 77.1) (end 89.875 77.1) (width 1) (layer "F.Cu") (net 6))
 (segment (start 93.05 83.13) (end 92.13 83.13) (width 0.2) (layer "F.Cu") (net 6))
 (segment (start 91.65 80.45) (end 91.975 80.125) (width 0.2) (layer "F.Cu") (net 6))
 (segment (start 92.15 80.3) (end 91.975 80.125) (width 0.2) (layer "F.Cu") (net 6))
 (segment (start 91.53 81.12) (end 91.53 82.59) (width 0.2) (layer "F.Cu") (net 6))
 (segment (start 91.65 81) (end 91.65 80.45) (width 0.2) (layer "F.Cu") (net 6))
 (segment (start 94.325 77.675) (end 94.4 77.6) (width 0.5) (layer "F.Cu") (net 6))
 (segment (start 92.325 77.675) (end 94.325 77.675) (width 0.5) (layer "F.Cu") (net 6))
 (segment (start 91.975 77.975) (end 92.25 77.7) (width 0.5) (layer "F.Cu") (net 6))
 (segment (start 89.875 77.1) (end 89.875 78.525) (width 1) (layer "F.Cu") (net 6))
 (segment (start 93.9 77.1) (end 92.15 77.1) (width 1) (layer "F.Cu") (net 6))
 (segment (start 92.13 83.13) (end 92.1 83.16) (width 0.2) (layer "F.Cu") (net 6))
 (segment (start 92.25 77.7) (end 92.3 77.7) (width 0.5) (layer "F.Cu") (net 6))
 (segment (start 91.53 82.59) (end 92.1 83.16) (width 0.2) (layer "F.Cu") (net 6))
 (segment (start 91.425 78.025) (end 90.4 79.05) (width 1) (layer "F.Cu") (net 6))
 (segment (start 92.15 77.1) (end 91.425 77.1) (width 1) (layer "F.Cu") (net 6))
 (segment (start 88.48 82.59) (end 89.05 83.16) (width 0.2) (layer "F.Cu") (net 2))
 (segment (start 88.65 81) (end 88.65 81.65) (width 0.2) (layer "F.Cu") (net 2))
 (segment (start 79.35 78.6) (end 85.025 78.6) (width 0.5) (layer "F.Cu") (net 2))
 (segment (start 86.725 77.125) (end 87.75 76.1) (width 0.5) (layer "F.Cu") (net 2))
 (segment (start 85.025 78.6) (end 86.5 77.125) (width 0.5) (layer "F.Cu") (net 2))
 (segment (start 90 82.21) (end 89.05 83.16) (width 0.2) (layer "F.Cu") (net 2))
 (segment (start 97.35 78.9) (end 98 79.55) (width 1) (layer "F.Cu") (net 2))
 (segment (start 83.3875 80.2375) (end 85.025 78.6) (width 0.5) (layer "F.Cu") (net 2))
 (segment (start 90 82.14) (end 90 82.21) (width 0.2) (layer "F.Cu") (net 2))
 (segment (start 79.35 80.6) (end 83.025 80.6) (width 0.5) (layer "F.Cu") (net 2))
 (segment (start 97.35 77.6) (end 97.35 78.9) (width 1) (layer "F.Cu") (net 2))
 (segment (start 89.05 83.16) (end 89.05 84.5) (width 0.5) (layer "F.Cu") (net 2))
 (segment (start 86.5 77.125) (end 86.725 77.125) (width 0.5) (layer "F.Cu") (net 2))
 (segment (start 96.3 79.75) (end 97.8 79.75) (width 1) (layer "F.Cu") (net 2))
 (segment (start 88.48 81.82) (end 88.48 82.59) (width 0.2) (layer "F.Cu") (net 2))
 (segment (start 90.15 81) (end 90.15 81.99) (width 0.2) (layer "F.Cu") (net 2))
 (segment (start 83.025 80.6) (end 83.3875 80.2375) (width 0.5) (layer "F.Cu") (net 2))
 (segment (start 89.05 83.16) (end 86.36 83.16) (width 0.5) (layer "F.Cu") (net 2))
 (segment (start 97.8 79.75) (end 98 79.55) (width 1) (layer "F.Cu") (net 2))
 (segment (start 88.65 81.65) (end 88.48 81.82) (width 0.2) (layer "F.Cu") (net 2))
 (segment (start 87.75 76.1) (end 95.85 76.1) (width 0.5) (layer "F.Cu") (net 2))
 (segment (start 90.15 81.99) (end 90 82.14) (width 0.2) (layer "F.Cu") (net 2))
 (segment (start 95.85 76.1) (end 97.35 77.6) (width 0.5) (layer "F.Cu") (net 2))
 (segment (start 86.36 83.16) (end 84.6 81.4) (width 0.5) (layer "F.Cu") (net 2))
 (via (at 84.6 81.4) (size 0.45) (drill 0.2) (layers "F.Cu" "B.Cu") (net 2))
 (via (at 83.3875 80.2375) (size 0.45) (drill 0.2) (layers "F.Cu" "B.Cu") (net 2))
 (via (at 89.05 84.5) (size 0.45) (drill 0.2) (layers "F.Cu" "B.Cu") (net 2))
 (segment (start 89.05 84.5) (end 79.4 84.5) (width 0.5) (layer "B.Cu") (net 2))
 (segment (start 84.55 81.4) (end 83.3875 80.2375) (width 0.5) (layer "B.Cu") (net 2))
 (segment (start 111.5 84.5) (end 89.05 84.5) (width 0.5) (layer "B.Cu") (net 2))
 (segment (start 79.4 84.5) (end 79.3 84.6) (width 0.5) (layer "B.Cu") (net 2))
 (segment (start 84.6 81.4) (end 84.55 81.4) (width 0.5) (layer "B.Cu") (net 2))
 (segment (start 90.65 81) (end 90.65 81.84) (width 0.2) (layer "F.Cu") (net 7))
 (segment (start 90.65 81.84) (end 90.95 82.14) (width 0.2) (layer "F.Cu") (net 7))
 (segment (start 90.95 82.21) (end 90 83.16) (width 0.2) (layer "F.Cu") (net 7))
 (segment (start 90.95 82.14) (end 90.95 82.21) (width 0.2) (layer "F.Cu") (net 7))
 (segment (start 86.55 80.86) (end 87.09 80.86) (width 0.2) (layer "F.Cu") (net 8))
 (segment (start 87.09 80.86) (end 87.25 80.7) (width 0.2) (layer "F.Cu") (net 8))
 (segment (start 87.5 79.3) (end 87.95 79.3) (width 0.2) (layer "F.Cu") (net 8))
 (segment (start 87.25 80.7) (end 87.25 79.55) (width 0.2) (layer "F.Cu") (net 8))
 (segment (start 87.25 79.55) (end 87.5 79.3) (width 0.2) (layer "F.Cu") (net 8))
 (segment (start 89.15 81) (end 89.15 82.04) (width 0.2) (layer "F.Cu") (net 10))
 (segment (start 89.15 82.04) (end 89.05 82.14) (width 0.2) (layer "F.Cu") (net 10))
 (segment (start 92.15 81) (end 92.15 82.09) (width 0.2) (layer "F.Cu") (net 9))
 (segment (start 92.15 82.09) (end 92.1 82.14) (width 0.2) (layer "F.Cu") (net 9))
 (segment (start 111.6 82.5) (end 79.5 82.5) (width 0.5) (layer "B.Cu") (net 4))
 (segment (start 79.5 82.5) (end 79.4 82.6) (width 0.5) (layer "B.Cu") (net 4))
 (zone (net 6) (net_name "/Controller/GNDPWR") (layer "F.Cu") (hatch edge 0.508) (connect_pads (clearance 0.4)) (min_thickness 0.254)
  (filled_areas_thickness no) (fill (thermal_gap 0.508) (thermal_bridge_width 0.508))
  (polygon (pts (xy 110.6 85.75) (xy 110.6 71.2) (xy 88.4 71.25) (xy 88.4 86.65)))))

